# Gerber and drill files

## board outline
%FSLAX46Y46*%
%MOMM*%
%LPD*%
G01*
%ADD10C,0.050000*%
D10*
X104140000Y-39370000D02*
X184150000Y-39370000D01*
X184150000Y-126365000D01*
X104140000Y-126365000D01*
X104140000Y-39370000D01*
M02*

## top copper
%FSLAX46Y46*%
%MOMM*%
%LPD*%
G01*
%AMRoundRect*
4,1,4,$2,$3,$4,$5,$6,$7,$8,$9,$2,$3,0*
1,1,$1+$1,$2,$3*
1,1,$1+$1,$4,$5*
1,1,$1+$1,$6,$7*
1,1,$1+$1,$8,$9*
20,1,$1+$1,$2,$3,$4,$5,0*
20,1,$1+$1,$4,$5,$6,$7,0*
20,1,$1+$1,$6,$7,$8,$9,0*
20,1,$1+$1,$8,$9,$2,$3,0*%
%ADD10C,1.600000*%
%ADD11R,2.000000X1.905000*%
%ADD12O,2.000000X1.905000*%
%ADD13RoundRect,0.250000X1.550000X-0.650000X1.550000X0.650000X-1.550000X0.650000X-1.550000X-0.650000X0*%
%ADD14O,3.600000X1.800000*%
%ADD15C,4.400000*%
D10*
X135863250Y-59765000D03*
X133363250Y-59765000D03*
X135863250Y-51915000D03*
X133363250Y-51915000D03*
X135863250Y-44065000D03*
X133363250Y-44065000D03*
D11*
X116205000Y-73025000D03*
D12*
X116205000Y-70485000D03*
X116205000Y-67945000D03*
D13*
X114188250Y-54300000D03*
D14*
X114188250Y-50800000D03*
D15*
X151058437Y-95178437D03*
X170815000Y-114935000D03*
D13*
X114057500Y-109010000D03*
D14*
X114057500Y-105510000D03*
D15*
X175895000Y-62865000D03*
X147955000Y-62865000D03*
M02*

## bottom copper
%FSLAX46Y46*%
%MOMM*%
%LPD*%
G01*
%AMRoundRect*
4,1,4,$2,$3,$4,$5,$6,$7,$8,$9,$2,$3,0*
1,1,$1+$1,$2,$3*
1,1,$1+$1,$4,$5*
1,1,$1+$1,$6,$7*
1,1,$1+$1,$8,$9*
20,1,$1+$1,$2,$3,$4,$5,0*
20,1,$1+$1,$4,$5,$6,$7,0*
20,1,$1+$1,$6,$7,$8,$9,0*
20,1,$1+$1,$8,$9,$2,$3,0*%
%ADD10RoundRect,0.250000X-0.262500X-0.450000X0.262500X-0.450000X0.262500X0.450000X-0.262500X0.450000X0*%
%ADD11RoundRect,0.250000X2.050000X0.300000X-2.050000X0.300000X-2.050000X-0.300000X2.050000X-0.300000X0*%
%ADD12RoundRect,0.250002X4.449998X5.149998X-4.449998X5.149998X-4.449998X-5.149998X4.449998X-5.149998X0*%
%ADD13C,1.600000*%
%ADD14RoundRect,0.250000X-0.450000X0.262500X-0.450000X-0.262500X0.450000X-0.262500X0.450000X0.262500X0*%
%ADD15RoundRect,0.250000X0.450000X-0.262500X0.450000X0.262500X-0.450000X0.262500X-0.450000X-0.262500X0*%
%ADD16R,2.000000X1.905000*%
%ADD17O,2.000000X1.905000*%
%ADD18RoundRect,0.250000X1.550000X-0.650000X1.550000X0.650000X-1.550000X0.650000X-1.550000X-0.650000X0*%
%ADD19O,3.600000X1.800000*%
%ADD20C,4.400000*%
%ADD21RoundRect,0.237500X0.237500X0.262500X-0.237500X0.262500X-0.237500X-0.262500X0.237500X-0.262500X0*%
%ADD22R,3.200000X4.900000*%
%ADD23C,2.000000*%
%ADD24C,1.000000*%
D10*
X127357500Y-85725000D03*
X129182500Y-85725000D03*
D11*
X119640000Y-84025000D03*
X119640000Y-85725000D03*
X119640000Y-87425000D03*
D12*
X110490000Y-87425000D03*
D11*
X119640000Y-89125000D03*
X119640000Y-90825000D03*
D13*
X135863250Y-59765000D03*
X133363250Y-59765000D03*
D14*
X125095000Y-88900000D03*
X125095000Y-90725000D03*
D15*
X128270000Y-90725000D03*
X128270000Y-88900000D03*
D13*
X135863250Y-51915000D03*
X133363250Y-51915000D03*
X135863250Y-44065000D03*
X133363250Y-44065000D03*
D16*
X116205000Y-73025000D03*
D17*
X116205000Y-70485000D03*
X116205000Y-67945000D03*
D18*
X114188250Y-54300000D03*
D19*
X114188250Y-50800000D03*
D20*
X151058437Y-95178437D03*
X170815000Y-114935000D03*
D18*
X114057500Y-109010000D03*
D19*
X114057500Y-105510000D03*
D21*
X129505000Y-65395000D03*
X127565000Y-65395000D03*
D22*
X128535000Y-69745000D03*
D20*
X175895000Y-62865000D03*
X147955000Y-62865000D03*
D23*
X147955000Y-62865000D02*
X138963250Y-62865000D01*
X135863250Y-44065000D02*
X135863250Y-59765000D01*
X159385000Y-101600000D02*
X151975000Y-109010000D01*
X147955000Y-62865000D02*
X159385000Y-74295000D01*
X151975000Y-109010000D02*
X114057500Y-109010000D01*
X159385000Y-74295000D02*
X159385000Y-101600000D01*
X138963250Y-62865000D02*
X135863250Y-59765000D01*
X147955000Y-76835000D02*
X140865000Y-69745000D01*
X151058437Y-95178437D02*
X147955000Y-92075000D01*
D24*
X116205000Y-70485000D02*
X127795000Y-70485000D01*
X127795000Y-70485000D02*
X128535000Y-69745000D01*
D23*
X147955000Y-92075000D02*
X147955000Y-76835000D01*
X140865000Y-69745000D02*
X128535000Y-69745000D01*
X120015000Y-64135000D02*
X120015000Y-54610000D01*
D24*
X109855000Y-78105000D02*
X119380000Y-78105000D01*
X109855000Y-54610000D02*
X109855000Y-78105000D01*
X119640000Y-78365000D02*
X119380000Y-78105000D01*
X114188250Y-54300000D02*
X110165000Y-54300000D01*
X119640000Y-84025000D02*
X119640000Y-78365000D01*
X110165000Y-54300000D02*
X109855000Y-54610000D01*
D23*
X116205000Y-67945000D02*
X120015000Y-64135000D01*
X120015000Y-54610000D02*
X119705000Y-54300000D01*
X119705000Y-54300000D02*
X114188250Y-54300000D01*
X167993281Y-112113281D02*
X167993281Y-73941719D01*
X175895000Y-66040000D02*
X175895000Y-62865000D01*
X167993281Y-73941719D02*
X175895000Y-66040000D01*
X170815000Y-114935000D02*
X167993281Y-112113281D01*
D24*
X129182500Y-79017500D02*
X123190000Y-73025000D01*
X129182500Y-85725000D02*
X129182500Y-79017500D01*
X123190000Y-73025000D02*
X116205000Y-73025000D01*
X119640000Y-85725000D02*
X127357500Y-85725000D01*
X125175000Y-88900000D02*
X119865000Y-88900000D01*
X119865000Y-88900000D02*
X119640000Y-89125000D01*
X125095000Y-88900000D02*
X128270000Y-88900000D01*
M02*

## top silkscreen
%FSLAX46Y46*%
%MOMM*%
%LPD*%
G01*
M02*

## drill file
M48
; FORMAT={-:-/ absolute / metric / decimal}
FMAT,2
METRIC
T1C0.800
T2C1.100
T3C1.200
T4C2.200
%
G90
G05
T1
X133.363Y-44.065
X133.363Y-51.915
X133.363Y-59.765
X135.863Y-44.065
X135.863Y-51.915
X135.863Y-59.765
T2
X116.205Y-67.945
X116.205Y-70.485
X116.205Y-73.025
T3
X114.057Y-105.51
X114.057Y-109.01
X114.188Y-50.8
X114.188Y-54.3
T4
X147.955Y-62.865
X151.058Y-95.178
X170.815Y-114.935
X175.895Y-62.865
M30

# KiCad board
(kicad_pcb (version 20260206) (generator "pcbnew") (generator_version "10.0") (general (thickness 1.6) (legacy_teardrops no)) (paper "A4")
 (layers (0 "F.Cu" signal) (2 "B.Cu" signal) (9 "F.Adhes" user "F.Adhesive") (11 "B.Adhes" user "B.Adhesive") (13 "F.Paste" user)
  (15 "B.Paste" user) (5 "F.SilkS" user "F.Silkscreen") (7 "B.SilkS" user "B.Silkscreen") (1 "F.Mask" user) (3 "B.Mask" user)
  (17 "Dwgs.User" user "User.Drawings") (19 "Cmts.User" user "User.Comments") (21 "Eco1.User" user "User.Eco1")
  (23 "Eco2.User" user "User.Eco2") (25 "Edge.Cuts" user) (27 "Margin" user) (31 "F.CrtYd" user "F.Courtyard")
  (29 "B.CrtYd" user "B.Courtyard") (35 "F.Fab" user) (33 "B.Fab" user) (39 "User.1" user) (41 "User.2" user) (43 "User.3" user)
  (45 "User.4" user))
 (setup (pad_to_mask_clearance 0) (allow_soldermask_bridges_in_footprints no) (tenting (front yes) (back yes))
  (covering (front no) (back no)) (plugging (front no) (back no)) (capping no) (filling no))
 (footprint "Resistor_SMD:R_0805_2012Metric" (layer "B.Cu") (at 128.27 85.725)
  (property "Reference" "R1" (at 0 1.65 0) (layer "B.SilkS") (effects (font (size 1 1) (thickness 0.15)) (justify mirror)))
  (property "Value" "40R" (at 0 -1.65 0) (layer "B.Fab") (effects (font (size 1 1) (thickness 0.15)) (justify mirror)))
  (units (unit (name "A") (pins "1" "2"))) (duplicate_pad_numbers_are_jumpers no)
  (pad "1" smd roundrect (at -0.9125 0) (size 1.025 1.4) (layers "B.Cu" "B.Mask" "B.Paste") (roundrect_rratio 0.243902) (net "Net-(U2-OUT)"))
  (pad "2" smd roundrect (at 0.9125 0) (size 1.025 1.4) (layers "B.Cu" "B.Mask" "B.Paste") (roundrect_rratio 0.243902) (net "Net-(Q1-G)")))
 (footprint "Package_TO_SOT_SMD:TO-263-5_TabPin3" (layer "B.Cu") (at 111.99 87.425 180)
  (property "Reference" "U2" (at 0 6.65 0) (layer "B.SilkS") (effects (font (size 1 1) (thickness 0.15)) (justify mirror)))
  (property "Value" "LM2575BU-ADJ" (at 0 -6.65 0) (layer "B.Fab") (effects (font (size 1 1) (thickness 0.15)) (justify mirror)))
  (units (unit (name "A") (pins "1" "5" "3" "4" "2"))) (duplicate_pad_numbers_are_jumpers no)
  (pad "" smd roundrect (at -0.925 -2.775 180) (size 4.55 5.25) (layers "B.Paste") (roundrect_rratio 0.054945))
  (pad "" smd roundrect (at -0.925 2.775 180) (size 4.55 5.25) (layers "B.Paste") (roundrect_rratio 0.054945))
  (pad "" smd roundrect (at 3.925 -2.775 180) (size 4.55 5.25) (layers "B.Paste") (roundrect_rratio 0.054945))
  (pad "" smd roundrect (at 3.925 2.775 180) (size 4.55 5.25) (layers "B.Paste") (roundrect_rratio 0.054945))
  (pad "1" smd roundrect (at -7.65 3.4 180) (size 4.6 1.1) (layers "B.Cu" "B.Mask" "B.Paste") (roundrect_rratio 0.227273) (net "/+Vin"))
  (pad "2" smd roundrect (at -7.65 1.7 180) (size 4.6 1.1) (layers "B.Cu" "B.Mask" "B.Paste") (roundrect_rratio 0.227273)
   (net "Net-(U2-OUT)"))
  (pad "3" smd roundrect (at -7.65 0 180) (size 4.6 1.1) (layers "B.Cu" "B.Mask" "B.Paste") (roundrect_rratio 0.227273) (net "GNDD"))
  (pad "3" smd roundrect (at 1.5 0 180) (size 9.4 10.8) (layers "B.Cu" "B.Mask") (roundrect_rratio 0.026596) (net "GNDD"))
  (pad "4" smd roundrect (at -7.65 -1.7 180) (size 4.6 1.1) (layers "B.Cu" "B.Mask" "B.Paste") (roundrect_rratio 0.227273)
   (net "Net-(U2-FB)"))
  (pad "5" smd roundrect (at -7.65 -3.4 180) (size 4.6 1.1) (layers "B.Cu" "B.Mask" "B.Paste") (roundrect_rratio 0.227273) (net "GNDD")))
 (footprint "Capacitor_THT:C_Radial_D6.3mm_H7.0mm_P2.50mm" (layer "B.Cu") (at 135.86325 59.765 180)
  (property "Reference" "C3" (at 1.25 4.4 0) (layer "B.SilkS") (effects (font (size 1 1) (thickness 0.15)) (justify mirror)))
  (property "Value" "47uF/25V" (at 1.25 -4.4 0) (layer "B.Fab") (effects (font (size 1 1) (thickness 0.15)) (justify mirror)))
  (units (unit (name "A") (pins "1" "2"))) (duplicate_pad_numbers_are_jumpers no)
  (pad "1" thru_hole circle (at 0 0 180) (size 1.6 1.6) (drill 0.8) (layers "*.Cu" "*.Mask") (remove_unused_layers no) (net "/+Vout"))
  (pad "2" thru_hole circle (at 2.5 0 180) (size 1.6 1.6) (drill 0.8) (layers "*.Cu" "*.Mask") (remove_unused_layers no) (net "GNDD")))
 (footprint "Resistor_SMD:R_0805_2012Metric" (layer "B.Cu") (at 125.095 89.8125 -90)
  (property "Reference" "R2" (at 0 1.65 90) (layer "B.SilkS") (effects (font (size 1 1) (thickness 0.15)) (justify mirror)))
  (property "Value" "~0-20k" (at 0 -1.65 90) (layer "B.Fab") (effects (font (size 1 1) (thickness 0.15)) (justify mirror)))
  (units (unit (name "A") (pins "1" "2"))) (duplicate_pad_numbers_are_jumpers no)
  (pad "1" smd roundrect (at -0.9125 0 270) (size 1.025 1.4) (layers "B.Cu" "B.Mask" "B.Paste") (roundrect_rratio 0.243902)
   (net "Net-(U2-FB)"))
  (pad "2" smd roundrect (at 0.9125 0 270) (size 1.025 1.4) (layers "B.Cu" "B.Mask" "B.Paste") (roundrect_rratio 0.243902) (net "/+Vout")))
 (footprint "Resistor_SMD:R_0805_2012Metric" (layer "B.Cu") (at 128.27 89.8125 90)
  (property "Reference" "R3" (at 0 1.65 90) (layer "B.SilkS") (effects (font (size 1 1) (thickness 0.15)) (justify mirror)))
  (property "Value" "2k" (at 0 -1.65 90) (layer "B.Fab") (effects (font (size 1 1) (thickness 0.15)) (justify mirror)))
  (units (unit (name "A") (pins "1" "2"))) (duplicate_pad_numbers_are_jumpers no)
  (pad "1" smd roundrect (at -0.9125 0 90) (size 1.025 1.4) (layers "B.Cu" "B.Mask" "B.Paste") (roundrect_rratio 0.243902) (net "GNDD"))
  (pad "2" smd roundrect (at 0.9125 0 90) (size 1.025 1.4) (layers "B.Cu" "B.Mask" "B.Paste") (roundrect_rratio 0.243902)
   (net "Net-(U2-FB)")))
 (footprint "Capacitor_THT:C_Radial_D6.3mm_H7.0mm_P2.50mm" (layer "B.Cu") (at 135.86325 51.915 180)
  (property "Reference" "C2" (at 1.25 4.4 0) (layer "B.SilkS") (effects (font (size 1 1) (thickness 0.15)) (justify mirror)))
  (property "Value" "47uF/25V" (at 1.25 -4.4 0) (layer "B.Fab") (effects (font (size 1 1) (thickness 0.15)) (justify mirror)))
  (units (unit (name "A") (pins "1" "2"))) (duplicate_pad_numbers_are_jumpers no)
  (pad "1" thru_hole circle (at 0 0 180) (size 1.6 1.6) (drill 0.8) (layers "*.Cu" "*.Mask") (remove_unused_layers no) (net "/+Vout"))
  (pad "2" thru_hole circle (at 2.5 0 180) (size 1.6 1.6) (drill 0.8) (layers "*.Cu" "*.Mask") (remove_unused_layers no) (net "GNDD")))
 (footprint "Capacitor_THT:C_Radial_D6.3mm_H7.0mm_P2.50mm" (layer "B.Cu") (at 135.86325 44.065 180)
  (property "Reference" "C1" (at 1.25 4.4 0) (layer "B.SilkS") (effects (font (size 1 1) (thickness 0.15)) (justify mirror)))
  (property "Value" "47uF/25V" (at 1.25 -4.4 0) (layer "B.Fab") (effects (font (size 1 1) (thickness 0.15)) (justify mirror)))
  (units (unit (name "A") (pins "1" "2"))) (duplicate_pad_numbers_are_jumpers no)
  (pad "1" thru_hole circle (at 0 0 180) (size 1.6 1.6) (drill 0.8) (layers "*.Cu" "*.Mask") (remove_unused_layers no) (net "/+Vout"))
  (pad "2" thru_hole circle (at 2.5 0 180) (size 1.6 1.6) (drill 0.8) (layers "*.Cu" "*.Mask") (remove_unused_layers no) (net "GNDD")))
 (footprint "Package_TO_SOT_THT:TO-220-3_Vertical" (layer "B.Cu") (at 116.205 73.025 90)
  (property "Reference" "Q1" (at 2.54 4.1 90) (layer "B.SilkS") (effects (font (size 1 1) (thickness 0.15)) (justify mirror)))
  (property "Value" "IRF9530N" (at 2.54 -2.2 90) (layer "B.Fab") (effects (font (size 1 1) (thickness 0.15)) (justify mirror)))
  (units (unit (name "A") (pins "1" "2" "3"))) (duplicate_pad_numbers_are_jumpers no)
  (pad "1" thru_hole rect (at 0 0 90) (size 1.905 2) (drill 1.1) (layers "*.Cu" "*.Mask") (remove_unused_layers no) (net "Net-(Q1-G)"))
  (pad "2" thru_hole oval (at 2.54 0 90) (size 1.905 2) (drill 1.1) (layers "*.Cu" "*.Mask") (remove_unused_layers no) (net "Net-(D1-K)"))
  (pad "3" thru_hole oval (at 5.08 0 90) (size 1.905 2) (drill 1.1) (layers "*.Cu" "*.Mask") (remove_unused_layers no) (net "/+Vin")))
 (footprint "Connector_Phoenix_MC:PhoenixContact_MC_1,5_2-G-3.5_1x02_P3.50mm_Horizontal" (layer "B.Cu") (at 114.18825 54.3 90)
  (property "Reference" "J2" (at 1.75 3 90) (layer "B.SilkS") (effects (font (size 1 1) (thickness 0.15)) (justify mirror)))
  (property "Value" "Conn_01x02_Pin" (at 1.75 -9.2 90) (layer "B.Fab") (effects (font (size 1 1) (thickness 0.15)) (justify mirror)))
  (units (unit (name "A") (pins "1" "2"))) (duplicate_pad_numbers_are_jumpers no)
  (pad "1" thru_hole roundrect (at 0 0 90) (size 1.8 3.6) (drill 1.2) (layers "*.Cu" "*.Mask") (remove_unused_layers no)
   (roundrect_rratio 0.138889) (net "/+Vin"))
  (pad "2" thru_hole oval (at 3.5 0 90) (size 1.8 3.6) (drill 1.2) (layers "*.Cu" "*.Mask") (remove_unused_layers no) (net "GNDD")))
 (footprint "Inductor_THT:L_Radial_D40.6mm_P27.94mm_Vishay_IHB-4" (layer "B.Cu") (at 151.058437 95.178437 -45)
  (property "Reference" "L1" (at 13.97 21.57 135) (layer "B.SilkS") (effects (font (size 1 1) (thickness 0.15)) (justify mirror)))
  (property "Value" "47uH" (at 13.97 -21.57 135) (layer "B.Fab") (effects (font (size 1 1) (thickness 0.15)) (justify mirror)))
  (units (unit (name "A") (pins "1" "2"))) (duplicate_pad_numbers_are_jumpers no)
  (pad "1" thru_hole circle (at 0 0 315) (size 4.4 4.4) (drill 2.2) (layers "*.Cu" "*.Mask") (remove_unused_layers no) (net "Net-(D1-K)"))
  (pad "2" thru_hole circle (at 27.939999 0 315) (size 4.4 4.4) (drill 2.2) (layers "*.Cu" "*.Mask") (remove_unused_layers no)
   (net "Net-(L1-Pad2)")))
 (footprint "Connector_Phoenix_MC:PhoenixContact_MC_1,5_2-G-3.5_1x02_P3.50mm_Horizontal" (layer "B.Cu") (at 114.0575 109.01 90)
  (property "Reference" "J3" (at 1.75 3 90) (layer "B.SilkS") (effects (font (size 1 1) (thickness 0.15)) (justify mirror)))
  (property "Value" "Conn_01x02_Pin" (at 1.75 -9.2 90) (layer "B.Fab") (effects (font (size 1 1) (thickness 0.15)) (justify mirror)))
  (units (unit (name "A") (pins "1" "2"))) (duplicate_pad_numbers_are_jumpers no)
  (pad "1" thru_hole roundrect (at 0 0 90) (size 1.8 3.6) (drill 1.2) (layers "*.Cu" "*.Mask") (remove_unused_layers no)
   (roundrect_rratio 0.138889) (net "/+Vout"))
  (pad "2" thru_hole oval (at 3.5 0 90) (size 1.8 3.6) (drill 1.2) (layers "*.Cu" "*.Mask") (remove_unused_layers no) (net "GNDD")))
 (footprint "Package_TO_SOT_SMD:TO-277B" (layer "B.Cu") (at 128.535 68.545 180)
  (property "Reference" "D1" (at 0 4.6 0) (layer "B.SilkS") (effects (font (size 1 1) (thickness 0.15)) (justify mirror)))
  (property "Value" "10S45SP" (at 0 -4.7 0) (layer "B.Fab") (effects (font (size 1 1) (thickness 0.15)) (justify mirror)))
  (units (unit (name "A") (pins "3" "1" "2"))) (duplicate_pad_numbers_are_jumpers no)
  (pad "" smd roundrect (at -0.9 -3 180) (size 1.3 1.2) (layers "B.Paste") (roundrect_rratio 0.25))
  (pad "" smd roundrect (at -0.9 -1.2 180) (size 1.3 1.2) (layers "B.Paste") (roundrect_rratio 0.25))
  (pad "" smd roundrect (at -0.9 0.6 180) (size 1.3 1.2) (layers "B.Paste") (roundrect_rratio 0.25))
  (pad "" smd roundrect (at 0.9 -3 180) (size 1.3 1.2) (layers "B.Paste") (roundrect_rratio 0.25))
  (pad "" smd roundrect (at 0.9 -1.2 180) (size 1.3 1.2) (layers "B.Paste") (roundrect_rratio 0.25))
  (pad "" smd roundrect (at 0.9 0.6 180) (size 1.3 1.2) (layers "B.Paste") (roundrect_rratio 0.25))
  (pad "1" smd roundrect (at -0.97 3.15 180) (size 0.95 1) (layers "B.Cu" "B.Mask" "B.Paste") (roundrect_rratio 0.25) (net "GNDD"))
  (pad "2" smd roundrect (at 0.97 3.15 180) (size 0.95 1) (layers "B.Cu" "B.Mask" "B.Paste") (roundrect_rratio 0.25) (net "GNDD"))
  (pad "3" smd rect (at 0 -1.2 180) (size 3.2 4.9) (layers "B.Cu" "B.Mask") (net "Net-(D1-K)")))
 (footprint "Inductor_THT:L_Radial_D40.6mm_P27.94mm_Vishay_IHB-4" (layer "B.Cu") (at 175.895 62.865 180)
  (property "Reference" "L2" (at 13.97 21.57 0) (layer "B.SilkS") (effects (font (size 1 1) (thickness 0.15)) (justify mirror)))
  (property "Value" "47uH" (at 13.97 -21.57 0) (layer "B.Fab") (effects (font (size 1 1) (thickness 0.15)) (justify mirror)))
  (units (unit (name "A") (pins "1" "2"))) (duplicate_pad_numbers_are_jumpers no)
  (pad "1" thru_hole circle (at 0 0 180) (size 4.4 4.4) (drill 2.2) (layers "*.Cu" "*.Mask") (remove_unused_layers no) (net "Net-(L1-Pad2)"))
  (pad "2" thru_hole circle (at 27.94 0 180) (size 4.4 4.4) (drill 2.2) (layers "*.Cu" "*.Mask") (remove_unused_layers no) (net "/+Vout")))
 (gr_rect (start 104.14 39.37) (end 184.15 126.365) (stroke (width 0.05) (type default)) (fill no) (layer "Edge.Cuts"))
 (segment (start 147.955 62.865) (end 138.96325 62.865) (width 2) (layer "B.Cu") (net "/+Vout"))
 (segment (start 135.86325 44.065) (end 135.86325 59.765) (width 2) (layer "B.Cu") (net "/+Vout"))
 (segment (start 159.385 101.6) (end 151.975 109.01) (width 2) (layer "B.Cu") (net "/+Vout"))
 (segment (start 147.955 62.865) (end 159.385 74.295) (width 2) (layer "B.Cu") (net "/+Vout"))
 (segment (start 151.975 109.01) (end 114.0575 109.01) (width 2) (layer "B.Cu") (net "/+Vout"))
 (segment (start 159.385 74.295) (end 159.385 101.6) (width 2) (layer "B.Cu") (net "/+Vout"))
 (segment (start 138.96325 62.865) (end 135.86325 59.765) (width 2) (layer "B.Cu") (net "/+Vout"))
 (segment (start 147.955 76.835) (end 140.865 69.745) (width 2) (layer "B.Cu") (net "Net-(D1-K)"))
 (segment (start 151.058437 95.178437) (end 147.955 92.075) (width 2) (layer "B.Cu") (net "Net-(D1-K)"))
 (segment (start 116.205 70.485) (end 127.795 70.485) (width 1) (layer "B.Cu") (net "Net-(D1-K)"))
 (segment (start 127.795 70.485) (end 128.535 69.745) (width 1) (layer "B.Cu") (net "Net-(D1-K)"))
 (segment (start 147.955 92.075) (end 147.955 76.835) (width 2) (layer "B.Cu") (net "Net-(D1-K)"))
 (segment (start 140.865 69.745) (end 128.535 69.745) (width 2) (layer "B.Cu") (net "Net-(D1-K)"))
 (segment (start 120.015 64.135) (end 120.015 54.61) (width 2) (layer "B.Cu") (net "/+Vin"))
 (segment (start 109.855 78.105) (end 119.38 78.105) (width 1) (layer "B.Cu") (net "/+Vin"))
 (segment (start 109.855 54.61) (end 109.855 78.105) (width 1) (layer "B.Cu") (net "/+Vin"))
 (segment (start 119.64 78.365) (end 119.38 78.105) (width 1) (layer "B.Cu") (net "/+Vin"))
 (segment (start 114.18825 54.3) (end 110.165 54.3) (width 1) (layer "B.Cu") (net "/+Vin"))
 (segment (start 119.64 84.025) (end 119.64 78.365) (width 1) (layer "B.Cu") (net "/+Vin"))
 (segment (start 110.165 54.3) (end 109.855 54.61) (width 1) (layer "B.Cu") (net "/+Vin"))
 (segment (start 116.205 67.945) (end 120.015 64.135) (width 2) (layer "B.Cu") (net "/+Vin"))
 (segment (start 120.015 54.61) (end 119.705 54.3) (width 2) (layer "B.Cu") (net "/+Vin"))
 (segment (start 119.705 54.3) (end 114.18825 54.3) (width 2) (layer "B.Cu") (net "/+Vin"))
 (segment (start 167.993281 112.113281) (end 167.993281 73.941719) (width 2) (layer "B.Cu") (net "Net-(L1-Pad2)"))
 (segment (start 175.895 66.04) (end 175.895 62.865) (width 2) (layer "B.Cu") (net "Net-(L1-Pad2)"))
 (segment (start 167.993281 73.941719) (end 175.895 66.04) (width 2) (layer "B.Cu") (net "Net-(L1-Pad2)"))
 (segment (start 170.815 114.935) (end 167.993281 112.113281) (width 2) (layer "B.Cu") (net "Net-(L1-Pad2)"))
 (segment (start 129.1825 79.0175) (end 123.19 73.025) (width 1) (layer "B.Cu") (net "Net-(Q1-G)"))
 (segment (start 129.1825 85.725) (end 129.1825 79.0175) (width 1) (layer "B.Cu") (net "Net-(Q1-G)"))
 (segment (start 123.19 73.025) (end 116.205 73.025) (width 1) (layer "B.Cu") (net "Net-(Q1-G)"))
 (segment (start 119.64 85.725) (end 127.3575 85.725) (width 1) (layer "B.Cu") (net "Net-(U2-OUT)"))
 (segment (start 125.175 88.9) (end 119.865 88.9) (width 1) (layer "B.Cu") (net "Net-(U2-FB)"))
 (segment (start 119.865 88.9) (end 119.64 89.125) (width 1) (layer "B.Cu") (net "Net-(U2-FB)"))
 (segment (start 125.095 88.9) (end 128.27 88.9) (width 1) (layer "B.Cu") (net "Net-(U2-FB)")))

